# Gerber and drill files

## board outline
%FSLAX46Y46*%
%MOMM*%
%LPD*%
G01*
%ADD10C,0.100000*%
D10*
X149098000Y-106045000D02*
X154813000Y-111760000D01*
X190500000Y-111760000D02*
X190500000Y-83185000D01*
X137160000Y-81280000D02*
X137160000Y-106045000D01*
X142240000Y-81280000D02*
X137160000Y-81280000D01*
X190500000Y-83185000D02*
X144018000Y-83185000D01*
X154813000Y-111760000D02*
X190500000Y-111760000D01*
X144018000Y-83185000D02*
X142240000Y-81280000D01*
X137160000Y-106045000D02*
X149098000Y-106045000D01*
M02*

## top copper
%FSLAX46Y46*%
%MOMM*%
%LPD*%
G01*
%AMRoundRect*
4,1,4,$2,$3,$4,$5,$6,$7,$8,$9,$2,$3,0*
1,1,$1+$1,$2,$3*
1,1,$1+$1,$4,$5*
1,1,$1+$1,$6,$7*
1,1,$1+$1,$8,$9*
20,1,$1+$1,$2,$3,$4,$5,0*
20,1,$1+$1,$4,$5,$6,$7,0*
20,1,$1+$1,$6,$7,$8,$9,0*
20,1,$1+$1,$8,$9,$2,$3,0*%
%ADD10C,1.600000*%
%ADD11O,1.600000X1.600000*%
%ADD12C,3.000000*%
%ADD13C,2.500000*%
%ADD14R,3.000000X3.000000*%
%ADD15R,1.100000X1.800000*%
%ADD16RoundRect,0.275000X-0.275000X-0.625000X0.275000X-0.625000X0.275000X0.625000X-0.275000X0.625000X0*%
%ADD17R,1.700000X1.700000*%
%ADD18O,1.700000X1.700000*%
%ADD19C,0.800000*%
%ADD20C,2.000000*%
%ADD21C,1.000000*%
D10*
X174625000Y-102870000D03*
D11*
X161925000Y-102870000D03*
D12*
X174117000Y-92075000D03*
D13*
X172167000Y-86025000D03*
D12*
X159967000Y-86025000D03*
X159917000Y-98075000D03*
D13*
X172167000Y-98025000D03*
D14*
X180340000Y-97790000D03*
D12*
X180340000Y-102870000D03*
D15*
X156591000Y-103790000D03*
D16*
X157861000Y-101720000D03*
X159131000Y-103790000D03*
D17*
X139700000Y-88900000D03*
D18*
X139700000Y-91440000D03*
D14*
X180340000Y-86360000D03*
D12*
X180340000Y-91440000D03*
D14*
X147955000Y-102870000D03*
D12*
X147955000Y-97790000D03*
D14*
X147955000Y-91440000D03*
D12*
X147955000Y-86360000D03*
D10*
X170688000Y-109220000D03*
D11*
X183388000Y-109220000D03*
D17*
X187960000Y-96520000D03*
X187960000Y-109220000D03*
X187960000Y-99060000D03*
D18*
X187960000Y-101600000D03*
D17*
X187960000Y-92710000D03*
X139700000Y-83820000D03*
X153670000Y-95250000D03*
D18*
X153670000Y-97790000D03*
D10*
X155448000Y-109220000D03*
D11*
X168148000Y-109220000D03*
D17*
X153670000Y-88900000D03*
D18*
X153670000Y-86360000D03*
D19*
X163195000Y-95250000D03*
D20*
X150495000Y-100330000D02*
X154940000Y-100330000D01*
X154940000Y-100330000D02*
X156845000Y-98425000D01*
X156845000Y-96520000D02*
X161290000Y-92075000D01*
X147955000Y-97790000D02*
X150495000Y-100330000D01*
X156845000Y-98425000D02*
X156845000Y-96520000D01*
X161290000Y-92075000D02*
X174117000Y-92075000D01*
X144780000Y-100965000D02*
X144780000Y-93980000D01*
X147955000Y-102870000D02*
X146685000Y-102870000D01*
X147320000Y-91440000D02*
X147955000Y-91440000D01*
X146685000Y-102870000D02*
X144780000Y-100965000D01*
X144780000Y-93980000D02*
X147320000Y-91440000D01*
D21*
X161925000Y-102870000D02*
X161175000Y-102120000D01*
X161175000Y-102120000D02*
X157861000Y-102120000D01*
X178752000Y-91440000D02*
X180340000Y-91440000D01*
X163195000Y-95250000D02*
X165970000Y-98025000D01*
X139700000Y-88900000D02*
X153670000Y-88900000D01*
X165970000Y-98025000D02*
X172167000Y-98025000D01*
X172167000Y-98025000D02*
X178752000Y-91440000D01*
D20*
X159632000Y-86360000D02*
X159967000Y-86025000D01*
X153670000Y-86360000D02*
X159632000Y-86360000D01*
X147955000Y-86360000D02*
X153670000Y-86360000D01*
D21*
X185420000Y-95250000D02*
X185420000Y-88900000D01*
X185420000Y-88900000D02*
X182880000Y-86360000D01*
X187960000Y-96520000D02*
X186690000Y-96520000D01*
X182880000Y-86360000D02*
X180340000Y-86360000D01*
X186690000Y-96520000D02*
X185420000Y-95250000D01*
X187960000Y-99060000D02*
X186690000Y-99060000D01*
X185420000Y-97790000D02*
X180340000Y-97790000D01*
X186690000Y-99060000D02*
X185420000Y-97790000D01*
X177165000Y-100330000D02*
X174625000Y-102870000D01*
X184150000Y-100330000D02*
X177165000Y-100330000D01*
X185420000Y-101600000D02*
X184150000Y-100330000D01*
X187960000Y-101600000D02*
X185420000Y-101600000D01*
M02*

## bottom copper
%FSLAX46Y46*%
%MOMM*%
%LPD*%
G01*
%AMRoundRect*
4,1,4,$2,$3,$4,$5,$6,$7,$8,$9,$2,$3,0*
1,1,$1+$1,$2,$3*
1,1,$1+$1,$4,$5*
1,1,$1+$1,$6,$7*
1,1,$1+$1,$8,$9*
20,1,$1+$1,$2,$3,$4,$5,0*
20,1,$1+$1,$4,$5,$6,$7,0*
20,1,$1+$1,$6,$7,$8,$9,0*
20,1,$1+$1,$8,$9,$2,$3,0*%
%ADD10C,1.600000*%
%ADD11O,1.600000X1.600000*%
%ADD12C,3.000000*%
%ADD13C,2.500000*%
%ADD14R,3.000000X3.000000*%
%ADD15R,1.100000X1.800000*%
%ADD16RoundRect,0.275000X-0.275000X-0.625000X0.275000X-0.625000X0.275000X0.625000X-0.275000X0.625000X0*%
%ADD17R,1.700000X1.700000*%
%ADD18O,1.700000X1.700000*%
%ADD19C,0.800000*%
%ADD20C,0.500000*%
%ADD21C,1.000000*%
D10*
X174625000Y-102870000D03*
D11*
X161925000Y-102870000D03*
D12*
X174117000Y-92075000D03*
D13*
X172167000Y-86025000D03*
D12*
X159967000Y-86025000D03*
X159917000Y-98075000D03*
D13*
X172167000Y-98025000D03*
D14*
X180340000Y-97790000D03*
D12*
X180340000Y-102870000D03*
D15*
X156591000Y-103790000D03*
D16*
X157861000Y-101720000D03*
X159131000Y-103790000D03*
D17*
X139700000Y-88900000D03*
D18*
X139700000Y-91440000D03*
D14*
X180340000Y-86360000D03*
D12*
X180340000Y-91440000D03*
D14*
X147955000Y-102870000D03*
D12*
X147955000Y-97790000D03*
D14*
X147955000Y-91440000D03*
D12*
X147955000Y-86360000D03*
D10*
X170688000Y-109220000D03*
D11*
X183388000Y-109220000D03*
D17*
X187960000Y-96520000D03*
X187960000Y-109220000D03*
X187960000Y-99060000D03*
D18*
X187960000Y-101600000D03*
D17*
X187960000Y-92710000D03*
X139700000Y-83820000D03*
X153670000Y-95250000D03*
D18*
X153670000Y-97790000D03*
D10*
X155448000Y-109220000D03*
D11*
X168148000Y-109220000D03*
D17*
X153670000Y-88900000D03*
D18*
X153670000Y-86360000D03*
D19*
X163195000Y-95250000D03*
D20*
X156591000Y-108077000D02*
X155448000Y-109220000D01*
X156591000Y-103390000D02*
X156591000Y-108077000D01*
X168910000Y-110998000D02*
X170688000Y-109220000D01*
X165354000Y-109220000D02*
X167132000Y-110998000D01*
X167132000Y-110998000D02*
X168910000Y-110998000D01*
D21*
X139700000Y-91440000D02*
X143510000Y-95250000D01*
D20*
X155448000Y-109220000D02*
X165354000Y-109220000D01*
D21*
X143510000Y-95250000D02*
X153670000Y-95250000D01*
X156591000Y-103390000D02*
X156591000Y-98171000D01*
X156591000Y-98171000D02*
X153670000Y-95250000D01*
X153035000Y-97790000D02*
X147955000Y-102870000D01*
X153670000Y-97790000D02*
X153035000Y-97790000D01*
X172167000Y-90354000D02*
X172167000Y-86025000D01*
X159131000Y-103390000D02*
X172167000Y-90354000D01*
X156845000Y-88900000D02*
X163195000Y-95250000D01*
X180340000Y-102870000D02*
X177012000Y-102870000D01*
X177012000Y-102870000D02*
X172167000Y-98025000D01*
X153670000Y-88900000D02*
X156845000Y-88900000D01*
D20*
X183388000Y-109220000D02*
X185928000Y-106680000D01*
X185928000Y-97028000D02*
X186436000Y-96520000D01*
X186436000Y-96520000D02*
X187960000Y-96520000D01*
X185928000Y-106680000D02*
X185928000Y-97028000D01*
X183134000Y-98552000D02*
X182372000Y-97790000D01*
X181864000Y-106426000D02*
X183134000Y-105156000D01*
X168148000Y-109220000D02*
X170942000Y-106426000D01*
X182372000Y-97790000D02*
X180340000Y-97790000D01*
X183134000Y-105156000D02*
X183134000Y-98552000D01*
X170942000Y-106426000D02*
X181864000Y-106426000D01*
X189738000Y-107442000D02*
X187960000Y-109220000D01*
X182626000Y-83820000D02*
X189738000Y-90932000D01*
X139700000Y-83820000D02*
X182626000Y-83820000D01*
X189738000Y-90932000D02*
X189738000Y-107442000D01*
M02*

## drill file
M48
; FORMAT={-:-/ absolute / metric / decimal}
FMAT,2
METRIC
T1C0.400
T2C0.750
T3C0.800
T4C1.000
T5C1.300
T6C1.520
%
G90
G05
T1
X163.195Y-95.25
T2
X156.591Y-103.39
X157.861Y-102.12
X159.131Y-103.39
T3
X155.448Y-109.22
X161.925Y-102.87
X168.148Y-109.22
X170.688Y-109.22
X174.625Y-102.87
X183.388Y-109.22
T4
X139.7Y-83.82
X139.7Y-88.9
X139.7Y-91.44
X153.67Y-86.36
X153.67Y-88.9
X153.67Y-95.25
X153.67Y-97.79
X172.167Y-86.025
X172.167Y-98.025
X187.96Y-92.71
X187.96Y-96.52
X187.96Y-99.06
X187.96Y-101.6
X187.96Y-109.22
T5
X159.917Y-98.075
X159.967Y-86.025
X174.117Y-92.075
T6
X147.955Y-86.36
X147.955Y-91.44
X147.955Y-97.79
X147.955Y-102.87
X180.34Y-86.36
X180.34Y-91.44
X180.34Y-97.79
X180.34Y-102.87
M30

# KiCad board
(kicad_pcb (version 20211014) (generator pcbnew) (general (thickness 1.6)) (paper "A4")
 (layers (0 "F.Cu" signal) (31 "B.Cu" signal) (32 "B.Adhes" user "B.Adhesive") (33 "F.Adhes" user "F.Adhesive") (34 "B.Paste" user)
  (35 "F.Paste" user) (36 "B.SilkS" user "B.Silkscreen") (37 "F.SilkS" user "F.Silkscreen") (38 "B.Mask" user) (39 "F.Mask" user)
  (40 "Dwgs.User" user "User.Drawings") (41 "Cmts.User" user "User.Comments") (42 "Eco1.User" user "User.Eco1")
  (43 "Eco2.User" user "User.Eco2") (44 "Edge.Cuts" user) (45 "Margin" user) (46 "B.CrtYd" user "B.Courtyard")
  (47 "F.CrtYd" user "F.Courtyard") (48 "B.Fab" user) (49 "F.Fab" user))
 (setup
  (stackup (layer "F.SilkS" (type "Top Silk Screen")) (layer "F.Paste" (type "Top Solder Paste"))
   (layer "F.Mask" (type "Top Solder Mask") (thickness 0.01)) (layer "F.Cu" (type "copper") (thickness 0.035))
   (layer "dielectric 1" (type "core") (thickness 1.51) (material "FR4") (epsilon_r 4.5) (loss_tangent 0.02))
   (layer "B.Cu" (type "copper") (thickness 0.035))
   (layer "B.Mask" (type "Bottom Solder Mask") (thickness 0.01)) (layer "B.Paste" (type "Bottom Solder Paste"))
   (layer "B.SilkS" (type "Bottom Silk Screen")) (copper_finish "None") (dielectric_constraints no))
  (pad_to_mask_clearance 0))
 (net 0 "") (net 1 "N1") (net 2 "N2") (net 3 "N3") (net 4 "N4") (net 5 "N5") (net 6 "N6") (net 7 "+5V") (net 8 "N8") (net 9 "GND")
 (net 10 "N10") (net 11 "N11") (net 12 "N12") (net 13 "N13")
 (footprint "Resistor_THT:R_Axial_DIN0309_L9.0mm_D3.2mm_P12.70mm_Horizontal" (layer "F.Cu") (at 174.625 102.87 180)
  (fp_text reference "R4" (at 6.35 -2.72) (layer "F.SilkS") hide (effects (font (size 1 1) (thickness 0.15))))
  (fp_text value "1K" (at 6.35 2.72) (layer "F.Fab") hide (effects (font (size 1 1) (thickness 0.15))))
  (pad "1" thru_hole circle locked (at 0 0 180) (size 1.6 1.6) (drill 0.8) (layers *.Cu *.Mask) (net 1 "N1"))
  (pad "2" thru_hole oval locked (at 12.7 0 180) (size 1.6 1.6) (drill 0.8) (layers *.Cu *.Mask) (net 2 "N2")))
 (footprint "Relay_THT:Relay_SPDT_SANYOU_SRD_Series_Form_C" (layer "F.Cu") (at 174.117 92.075 180)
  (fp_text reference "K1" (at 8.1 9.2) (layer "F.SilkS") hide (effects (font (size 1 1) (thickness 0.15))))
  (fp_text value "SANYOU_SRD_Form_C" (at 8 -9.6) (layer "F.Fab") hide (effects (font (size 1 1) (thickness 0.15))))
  (pad "1" thru_hole circle locked (at 0 0 270) (size 3 3) (drill 1.3) (layers *.Cu *.Mask) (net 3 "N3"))
  (pad "2" thru_hole circle locked (at 1.95 6.05 270) (size 2.5 2.5) (drill 1) (layers *.Cu *.Mask) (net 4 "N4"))
  (pad "3" thru_hole circle locked (at 14.15 6.05 270) (size 3 3) (drill 1.3) (layers *.Cu *.Mask) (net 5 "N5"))
  (pad "4" thru_hole circle locked (at 14.2 -6 270) (size 3 3) (drill 1.3) (layers *.Cu *.Mask) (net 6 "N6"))
  (pad "5" thru_hole circle locked (at 1.95 -5.95 270) (size 2.5 2.5) (drill 1) (layers *.Cu *.Mask) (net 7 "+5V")))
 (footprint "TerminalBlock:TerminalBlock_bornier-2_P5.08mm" (layer "F.Cu") (at 180.34 97.79 -90)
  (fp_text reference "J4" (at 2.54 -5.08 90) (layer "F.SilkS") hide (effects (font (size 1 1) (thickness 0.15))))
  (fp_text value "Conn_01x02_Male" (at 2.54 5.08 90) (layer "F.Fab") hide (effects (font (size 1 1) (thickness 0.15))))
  (pad "1" thru_hole rect locked (at 0 0 270) (size 3 3) (drill 1.52) (layers *.Cu *.Mask) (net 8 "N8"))
  (pad "2" thru_hole circle locked (at 5.08 0 270) (size 3 3) (drill 1.52) (layers *.Cu *.Mask) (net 7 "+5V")))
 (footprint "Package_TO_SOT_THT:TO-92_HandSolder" (layer "F.Cu") (at 156.591 103.39)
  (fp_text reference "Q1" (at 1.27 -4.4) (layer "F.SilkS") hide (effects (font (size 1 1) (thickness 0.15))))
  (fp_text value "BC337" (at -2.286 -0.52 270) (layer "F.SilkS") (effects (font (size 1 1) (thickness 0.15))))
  (pad "1" thru_hole rect locked (at 0 0) (size 1.1 1.8) (drill 0.75 (offset 0 0.4)) (layers *.Cu *.Mask) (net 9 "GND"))
  (pad "2" thru_hole roundrect locked (at 1.27 -1.27) (size 1.1 1.8) (drill 0.75 (offset 0 -0.4)) (layers *.Cu *.Mask)
   (roundrect_rratio 0.25) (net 2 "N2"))
  (pad "3" thru_hole roundrect locked (at 2.54 0) (size 1.1 1.8) (drill 0.75 (offset 0 0.4)) (layers *.Cu *.Mask) (roundrect_rratio 0.25)
   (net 4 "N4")))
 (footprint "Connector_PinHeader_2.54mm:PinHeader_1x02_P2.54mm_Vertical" (layer "F.Cu") (at 139.7 88.9)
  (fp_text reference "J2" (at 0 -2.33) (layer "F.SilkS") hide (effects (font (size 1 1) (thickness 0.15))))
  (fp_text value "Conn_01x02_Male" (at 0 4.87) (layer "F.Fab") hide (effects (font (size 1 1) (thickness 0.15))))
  (pad "1" thru_hole rect locked (at 0 0) (size 1.7 1.7) (drill 1) (layers *.Cu *.Mask) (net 7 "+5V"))
  (pad "2" thru_hole oval locked (at 0 2.54) (size 1.7 1.7) (drill 1) (layers *.Cu *.Mask) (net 9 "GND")))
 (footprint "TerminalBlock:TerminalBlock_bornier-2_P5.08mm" (layer "F.Cu") (at 180.34 86.36 -90)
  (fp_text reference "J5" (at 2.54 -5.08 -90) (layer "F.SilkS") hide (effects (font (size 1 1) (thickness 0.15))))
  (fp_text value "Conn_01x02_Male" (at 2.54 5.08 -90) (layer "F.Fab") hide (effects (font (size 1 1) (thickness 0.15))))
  (pad "1" thru_hole rect locked (at 0 0 270) (size 3 3) (drill 1.52) (layers *.Cu *.Mask) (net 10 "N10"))
  (pad "2" thru_hole circle locked (at 5.08 0 270) (size 3 3) (drill 1.52) (layers *.Cu *.Mask) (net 7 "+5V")))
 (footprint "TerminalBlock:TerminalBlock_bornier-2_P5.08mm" (layer "F.Cu") (at 147.955 102.87 90)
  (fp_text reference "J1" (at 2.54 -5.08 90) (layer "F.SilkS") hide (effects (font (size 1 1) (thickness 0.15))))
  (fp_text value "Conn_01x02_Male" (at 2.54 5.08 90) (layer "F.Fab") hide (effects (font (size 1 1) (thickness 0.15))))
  (pad "1" thru_hole rect locked (at 0 0 90) (size 3 3) (drill 1.52) (layers *.Cu *.Mask) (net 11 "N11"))
  (pad "2" thru_hole circle locked (at 5.08 0 90) (size 3 3) (drill 1.52) (layers *.Cu *.Mask) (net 3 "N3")))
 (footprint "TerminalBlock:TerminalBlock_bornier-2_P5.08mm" (layer "F.Cu") (at 147.955 91.44 90)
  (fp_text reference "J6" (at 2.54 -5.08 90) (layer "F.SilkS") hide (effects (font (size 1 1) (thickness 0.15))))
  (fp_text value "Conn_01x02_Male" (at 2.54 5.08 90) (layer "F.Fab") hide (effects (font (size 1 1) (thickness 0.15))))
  (pad "1" thru_hole rect locked (at 0 0 90) (size 3 3) (drill 1.52) (layers *.Cu *.Mask) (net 11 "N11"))
  (pad "2" thru_hole circle locked (at 5.08 0 90) (size 3 3) (drill 1.52) (layers *.Cu *.Mask) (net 5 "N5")))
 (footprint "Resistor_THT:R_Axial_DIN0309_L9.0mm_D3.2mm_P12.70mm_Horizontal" (layer "F.Cu") (at 170.688 109.22)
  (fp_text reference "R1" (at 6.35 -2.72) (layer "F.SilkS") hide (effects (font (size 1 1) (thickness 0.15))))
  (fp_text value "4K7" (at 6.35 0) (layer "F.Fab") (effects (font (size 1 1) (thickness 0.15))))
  (pad "1" thru_hole circle (at 0 0) (size 1.6 1.6) (drill 0.8) (layers *.Cu *.Mask) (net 9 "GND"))
  (pad "2" thru_hole oval (at 12.7 0) (size 1.6 1.6) (drill 0.8) (layers *.Cu *.Mask) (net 10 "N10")))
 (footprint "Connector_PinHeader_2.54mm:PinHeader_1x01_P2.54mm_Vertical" (layer "F.Cu") (at 187.96 96.52)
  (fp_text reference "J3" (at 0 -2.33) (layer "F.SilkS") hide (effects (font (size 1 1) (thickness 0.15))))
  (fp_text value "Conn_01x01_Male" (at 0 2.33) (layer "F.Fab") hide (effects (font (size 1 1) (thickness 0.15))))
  (pad "1" thru_hole rect (at 0 0) (size 1.7 1.7) (drill 1) (layers *.Cu *.Mask) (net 10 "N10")))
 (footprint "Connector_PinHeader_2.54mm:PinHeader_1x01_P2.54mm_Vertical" (layer "F.Cu") (at 187.96 109.22)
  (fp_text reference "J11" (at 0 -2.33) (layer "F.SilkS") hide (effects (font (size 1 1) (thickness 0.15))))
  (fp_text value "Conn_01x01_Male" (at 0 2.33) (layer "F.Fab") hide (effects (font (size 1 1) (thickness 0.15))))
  (pad "1" thru_hole rect (at 0 0) (size 1.7 1.7) (drill 1) (layers *.Cu *.Mask) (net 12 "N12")))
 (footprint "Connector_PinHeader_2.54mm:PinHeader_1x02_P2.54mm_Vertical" (layer "F.Cu") (at 187.96 99.06)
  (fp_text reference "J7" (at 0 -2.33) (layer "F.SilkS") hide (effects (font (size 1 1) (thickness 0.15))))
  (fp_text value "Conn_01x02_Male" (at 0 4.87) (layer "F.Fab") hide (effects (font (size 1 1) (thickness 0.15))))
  (pad "1" thru_hole rect (at 0 0) (size 1.7 1.7) (drill 1) (layers *.Cu *.Mask) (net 8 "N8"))
  (pad "2" thru_hole oval (at 0 2.54) (size 1.7 1.7) (drill 1) (layers *.Cu *.Mask) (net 1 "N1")))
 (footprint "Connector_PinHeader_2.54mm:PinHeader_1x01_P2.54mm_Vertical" (layer "F.Cu") (at 187.96 92.71)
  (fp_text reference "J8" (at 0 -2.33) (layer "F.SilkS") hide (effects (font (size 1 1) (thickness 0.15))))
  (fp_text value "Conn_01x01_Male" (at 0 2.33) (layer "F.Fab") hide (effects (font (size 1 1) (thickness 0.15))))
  (pad "1" thru_hole rect (at 0 0) (size 1.7 1.7) (drill 1) (layers *.Cu *.Mask) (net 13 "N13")))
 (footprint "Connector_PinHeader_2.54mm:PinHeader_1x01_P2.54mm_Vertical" (layer "F.Cu") (at 139.7 83.82)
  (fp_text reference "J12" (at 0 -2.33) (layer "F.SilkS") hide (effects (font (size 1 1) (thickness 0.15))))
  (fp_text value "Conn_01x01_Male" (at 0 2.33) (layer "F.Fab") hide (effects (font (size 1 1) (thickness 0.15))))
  (pad "1" thru_hole rect (at 0 0) (size 1.7 1.7) (drill 1) (layers *.Cu *.Mask) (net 12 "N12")))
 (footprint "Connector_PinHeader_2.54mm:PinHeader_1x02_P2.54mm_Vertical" (layer "F.Cu") (at 153.67 95.25)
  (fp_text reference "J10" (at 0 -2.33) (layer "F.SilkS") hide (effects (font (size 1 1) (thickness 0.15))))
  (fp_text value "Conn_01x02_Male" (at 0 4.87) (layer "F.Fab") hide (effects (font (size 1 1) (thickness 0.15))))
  (pad "1" thru_hole rect (at 0 0) (size 1.7 1.7) (drill 1) (layers *.Cu *.Mask) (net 9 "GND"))
  (pad "2" thru_hole oval (at 0 2.54) (size 1.7 1.7) (drill 1) (layers *.Cu *.Mask) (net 11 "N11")))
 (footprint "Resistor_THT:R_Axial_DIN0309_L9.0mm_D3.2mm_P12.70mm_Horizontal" (layer "F.Cu") (at 155.448 109.22)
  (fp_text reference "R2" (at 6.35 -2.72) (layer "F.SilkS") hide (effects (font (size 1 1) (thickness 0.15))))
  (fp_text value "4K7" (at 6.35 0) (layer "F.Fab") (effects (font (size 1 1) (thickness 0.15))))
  (pad "1" thru_hole circle (at 0 0) (size 1.6 1.6) (drill 0.8) (layers *.Cu *.Mask) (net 9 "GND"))
  (pad "2" thru_hole oval (at 12.7 0) (size 1.6 1.6) (drill 0.8) (layers *.Cu *.Mask) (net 8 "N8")))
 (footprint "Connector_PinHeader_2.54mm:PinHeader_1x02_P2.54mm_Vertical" (layer "F.Cu") (at 153.67 88.9 180)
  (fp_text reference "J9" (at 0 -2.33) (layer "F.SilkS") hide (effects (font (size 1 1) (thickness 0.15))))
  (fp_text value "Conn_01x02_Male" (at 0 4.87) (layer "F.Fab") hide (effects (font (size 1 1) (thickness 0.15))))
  (pad "1" thru_hole rect (at 0 0 180) (size 1.7 1.7) (drill 1) (layers *.Cu *.Mask) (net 7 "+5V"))
  (pad "2" thru_hole oval (at 0 2.54 180) (size 1.7 1.7) (drill 1) (layers *.Cu *.Mask) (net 5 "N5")))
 (gr_line (start 149.098 106.045) (end 154.813 111.76) (layer "Edge.Cuts") (width 0.1))
 (gr_line (start 190.5 111.76) (end 190.5 83.185) (layer "Edge.Cuts") (width 0.1))
 (gr_line (start 137.16 81.28) (end 137.16 106.045) (layer "Edge.Cuts") (width 0.1))
 (gr_line (start 142.24 81.28) (end 137.16 81.28) (layer "Edge.Cuts") (width 0.1))
 (gr_line (start 190.5 83.185) (end 144.018 83.185) (layer "Edge.Cuts") (width 0.1))
 (gr_line (start 154.813 111.76) (end 190.5 111.76) (layer "Edge.Cuts") (width 0.1))
 (gr_line (start 144.018 83.185) (end 142.24 81.28) (layer "Edge.Cuts") (width 0.1))
 (gr_line (start 137.16 106.045) (end 149.098 106.045) (layer "Edge.Cuts") (width 0.1))
 (segment (start 156.591 108.077) (end 155.448 109.22) (width 0.5) (layer "B.Cu") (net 9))
 (segment (start 156.591 103.39) (end 156.591 108.077) (width 0.5) (layer "B.Cu") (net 9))
 (segment (start 168.91 110.998) (end 170.688 109.22) (width 0.5) (layer "B.Cu") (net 9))
 (segment (start 165.354 109.22) (end 167.132 110.998) (width 0.5) (layer "B.Cu") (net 9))
 (segment (start 167.132 110.998) (end 168.91 110.998) (width 0.5) (layer "B.Cu") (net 9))
 (segment (start 139.7 91.44) (end 143.51 95.25) (width 1) (layer "B.Cu") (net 9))
 (segment (start 155.448 109.22) (end 165.354 109.22) (width 0.5) (layer "B.Cu") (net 9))
 (segment (start 143.51 95.25) (end 153.67 95.25) (width 1) (layer "B.Cu") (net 9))
 (segment (start 156.591 103.39) (end 156.591 98.171) (width 1) (layer "B.Cu") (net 9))
 (segment (start 156.591 98.171) (end 153.67 95.25) (width 1) (layer "B.Cu") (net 9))
 (segment (start 150.495 100.33) (end 154.94 100.33) (width 2) (layer "F.Cu") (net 3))
 (segment (start 154.94 100.33) (end 156.845 98.425) (width 2) (layer "F.Cu") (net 3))
 (segment (start 156.845 96.52) (end 161.29 92.075) (width 2) (layer "F.Cu") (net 3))
 (segment (start 147.955 97.79) (end 150.495 100.33) (width 2) (layer "F.Cu") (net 3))
 (segment (start 156.845 98.425) (end 156.845 96.52) (width 2) (layer "F.Cu") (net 3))
 (segment (start 161.29 92.075) (end 174.117 92.075) (width 2) (layer "F.Cu") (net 3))
 (segment (start 144.78 100.965) (end 144.78 93.98) (width 2) (layer "F.Cu") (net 11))
 (segment (start 147.955 102.87) (end 146.685 102.87) (width 2) (layer "F.Cu") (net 11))
 (segment (start 147.32 91.44) (end 147.955 91.44) (width 2) (layer "F.Cu") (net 11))
 (segment (start 146.685 102.87) (end 144.78 100.965) (width 2) (layer "F.Cu") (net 11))
 (segment (start 144.78 93.98) (end 147.32 91.44) (width 2) (layer "F.Cu") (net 11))
 (segment (start 153.035 97.79) (end 147.955 102.87) (width 1) (layer "B.Cu") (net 11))
 (segment (start 153.67 97.79) (end 153.035 97.79) (width 1) (layer "B.Cu") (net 11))
 (segment (start 172.167 90.354) (end 172.167 86.025) (width 1) (layer "B.Cu") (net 4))
 (segment (start 159.131 103.39) (end 172.167 90.354) (width 1) (layer "B.Cu") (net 4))
 (segment (start 161.925 102.87) (end 161.175 102.12) (width 1) (layer "F.Cu") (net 2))
 (segment (start 161.175 102.12) (end 157.861 102.12) (width 1) (layer "F.Cu") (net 2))
 (segment (start 178.752 91.44) (end 180.34 91.44) (width 1) (layer "F.Cu") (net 7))
 (segment (start 163.195 95.25) (end 165.97 98.025) (width 1) (layer "F.Cu") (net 7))
 (segment (start 139.7 88.9) (end 153.67 88.9) (width 1) (layer "F.Cu") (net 7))
 (segment (start 165.97 98.025) (end 172.167 98.025) (width 1) (layer "F.Cu") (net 7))
 (segment (start 172.167 98.025) (end 178.752 91.44) (width 1) (layer "F.Cu") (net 7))
 (via (at 163.195 95.25) (size 0.8) (drill 0.4) (layers "F.Cu" "B.Cu") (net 7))
 (segment (start 156.845 88.9) (end 163.195 95.25) (width 1) (layer "B.Cu") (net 7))
 (segment (start 180.34 102.87) (end 177.012 102.87) (width 1) (layer "B.Cu") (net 7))
 (segment (start 177.012 102.87) (end 172.167 98.025) (width 1) (layer "B.Cu") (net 7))
 (segment (start 153.67 88.9) (end 156.845 88.9) (width 1) (layer "B.Cu") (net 7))
 (segment (start 159.632 86.36) (end 159.967 86.025) (width 2) (layer "F.Cu") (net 5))
 (segment (start 153.67 86.36) (end 159.632 86.36) (width 2) (layer "F.Cu") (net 5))
 (segment (start 147.955 86.36) (end 153.67 86.36) (width 2) (layer "F.Cu") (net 5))
 (segment (start 185.42 95.25) (end 185.42 88.9) (width 1) (layer "F.Cu") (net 10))
 (segment (start 185.42 88.9) (end 182.88 86.36) (width 1) (layer "F.Cu") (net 10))
 (segment (start 187.96 96.52) (end 186.69 96.52) (width 1) (layer "F.Cu") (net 10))
 (segment (start 182.88 86.36) (end 180.34 86.36) (width 1) (layer "F.Cu") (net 10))
 (segment (start 186.69 96.52) (end 185.42 95.25) (width 1) (layer "F.Cu") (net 10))
 (segment (start 183.388 109.22) (end 185.928 106.68) (width 0.5) (layer "B.Cu") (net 10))
 (segment (start 185.928 97.028) (end 186.436 96.52) (width 0.5) (layer "B.Cu") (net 10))
 (segment (start 186.436 96.52) (end 187.96 96.52) (width 0.5) (layer "B.Cu") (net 10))
 (segment (start 185.928 106.68) (end 185.928 97.028) (width 0.5) (layer "B.Cu") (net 10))
 (segment (start 187.96 99.06) (end 186.69 99.06) (width 1) (layer "F.Cu") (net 8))
 (segment (start 185.42 97.79) (end 180.34 97.79) (width 1) (layer "F.Cu") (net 8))
 (segment (start 186.69 99.06) (end 185.42 97.79) (width 1) (layer "F.Cu") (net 8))
 (segment (start 183.134 98.552) (end 182.372 97.79) (width 0.5) (layer "B.Cu") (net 8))
 (segment (start 181.864 106.426) (end 183.134 105.156) (width 0.5) (layer "B.Cu") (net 8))
 (segment (start 168.148 109.22) (end 170.942 106.426) (width 0.5) (layer "B.Cu") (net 8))
 (segment (start 182.372 97.79) (end 180.34 97.79) (width 0.5) (layer "B.Cu") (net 8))
 (segment (start 183.134 105.156) (end 183.134 98.552) (width 0.5) (layer "B.Cu") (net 8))
 (segment (start 170.942 106.426) (end 181.864 106.426) (width 0.5) (layer "B.Cu") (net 8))
 (segment (start 177.165 100.33) (end 174.625 102.87) (width 1) (layer "F.Cu") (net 1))
 (segment (start 184.15 100.33) (end 177.165 100.33) (width 1) (layer "F.Cu") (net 1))
 (segment (start 185.42 101.6) (end 184.15 100.33) (width 1) (layer "F.Cu") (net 1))
 (segment (start 187.96 101.6) (end 185.42 101.6) (width 1) (layer "F.Cu") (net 1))
 (segment (start 189.738 107.442) (end 187.96 109.22) (width 0.5) (layer "B.Cu") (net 12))
 (segment (start 182.626 83.82) (end 189.738 90.932) (width 0.5) (layer "B.Cu") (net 12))
 (segment (start 139.7 83.82) (end 182.626 83.82) (width 0.5) (layer "B.Cu") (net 12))
 (segment (start 189.738 90.932) (end 189.738 107.442) (width 0.5) (layer "B.Cu") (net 12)))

